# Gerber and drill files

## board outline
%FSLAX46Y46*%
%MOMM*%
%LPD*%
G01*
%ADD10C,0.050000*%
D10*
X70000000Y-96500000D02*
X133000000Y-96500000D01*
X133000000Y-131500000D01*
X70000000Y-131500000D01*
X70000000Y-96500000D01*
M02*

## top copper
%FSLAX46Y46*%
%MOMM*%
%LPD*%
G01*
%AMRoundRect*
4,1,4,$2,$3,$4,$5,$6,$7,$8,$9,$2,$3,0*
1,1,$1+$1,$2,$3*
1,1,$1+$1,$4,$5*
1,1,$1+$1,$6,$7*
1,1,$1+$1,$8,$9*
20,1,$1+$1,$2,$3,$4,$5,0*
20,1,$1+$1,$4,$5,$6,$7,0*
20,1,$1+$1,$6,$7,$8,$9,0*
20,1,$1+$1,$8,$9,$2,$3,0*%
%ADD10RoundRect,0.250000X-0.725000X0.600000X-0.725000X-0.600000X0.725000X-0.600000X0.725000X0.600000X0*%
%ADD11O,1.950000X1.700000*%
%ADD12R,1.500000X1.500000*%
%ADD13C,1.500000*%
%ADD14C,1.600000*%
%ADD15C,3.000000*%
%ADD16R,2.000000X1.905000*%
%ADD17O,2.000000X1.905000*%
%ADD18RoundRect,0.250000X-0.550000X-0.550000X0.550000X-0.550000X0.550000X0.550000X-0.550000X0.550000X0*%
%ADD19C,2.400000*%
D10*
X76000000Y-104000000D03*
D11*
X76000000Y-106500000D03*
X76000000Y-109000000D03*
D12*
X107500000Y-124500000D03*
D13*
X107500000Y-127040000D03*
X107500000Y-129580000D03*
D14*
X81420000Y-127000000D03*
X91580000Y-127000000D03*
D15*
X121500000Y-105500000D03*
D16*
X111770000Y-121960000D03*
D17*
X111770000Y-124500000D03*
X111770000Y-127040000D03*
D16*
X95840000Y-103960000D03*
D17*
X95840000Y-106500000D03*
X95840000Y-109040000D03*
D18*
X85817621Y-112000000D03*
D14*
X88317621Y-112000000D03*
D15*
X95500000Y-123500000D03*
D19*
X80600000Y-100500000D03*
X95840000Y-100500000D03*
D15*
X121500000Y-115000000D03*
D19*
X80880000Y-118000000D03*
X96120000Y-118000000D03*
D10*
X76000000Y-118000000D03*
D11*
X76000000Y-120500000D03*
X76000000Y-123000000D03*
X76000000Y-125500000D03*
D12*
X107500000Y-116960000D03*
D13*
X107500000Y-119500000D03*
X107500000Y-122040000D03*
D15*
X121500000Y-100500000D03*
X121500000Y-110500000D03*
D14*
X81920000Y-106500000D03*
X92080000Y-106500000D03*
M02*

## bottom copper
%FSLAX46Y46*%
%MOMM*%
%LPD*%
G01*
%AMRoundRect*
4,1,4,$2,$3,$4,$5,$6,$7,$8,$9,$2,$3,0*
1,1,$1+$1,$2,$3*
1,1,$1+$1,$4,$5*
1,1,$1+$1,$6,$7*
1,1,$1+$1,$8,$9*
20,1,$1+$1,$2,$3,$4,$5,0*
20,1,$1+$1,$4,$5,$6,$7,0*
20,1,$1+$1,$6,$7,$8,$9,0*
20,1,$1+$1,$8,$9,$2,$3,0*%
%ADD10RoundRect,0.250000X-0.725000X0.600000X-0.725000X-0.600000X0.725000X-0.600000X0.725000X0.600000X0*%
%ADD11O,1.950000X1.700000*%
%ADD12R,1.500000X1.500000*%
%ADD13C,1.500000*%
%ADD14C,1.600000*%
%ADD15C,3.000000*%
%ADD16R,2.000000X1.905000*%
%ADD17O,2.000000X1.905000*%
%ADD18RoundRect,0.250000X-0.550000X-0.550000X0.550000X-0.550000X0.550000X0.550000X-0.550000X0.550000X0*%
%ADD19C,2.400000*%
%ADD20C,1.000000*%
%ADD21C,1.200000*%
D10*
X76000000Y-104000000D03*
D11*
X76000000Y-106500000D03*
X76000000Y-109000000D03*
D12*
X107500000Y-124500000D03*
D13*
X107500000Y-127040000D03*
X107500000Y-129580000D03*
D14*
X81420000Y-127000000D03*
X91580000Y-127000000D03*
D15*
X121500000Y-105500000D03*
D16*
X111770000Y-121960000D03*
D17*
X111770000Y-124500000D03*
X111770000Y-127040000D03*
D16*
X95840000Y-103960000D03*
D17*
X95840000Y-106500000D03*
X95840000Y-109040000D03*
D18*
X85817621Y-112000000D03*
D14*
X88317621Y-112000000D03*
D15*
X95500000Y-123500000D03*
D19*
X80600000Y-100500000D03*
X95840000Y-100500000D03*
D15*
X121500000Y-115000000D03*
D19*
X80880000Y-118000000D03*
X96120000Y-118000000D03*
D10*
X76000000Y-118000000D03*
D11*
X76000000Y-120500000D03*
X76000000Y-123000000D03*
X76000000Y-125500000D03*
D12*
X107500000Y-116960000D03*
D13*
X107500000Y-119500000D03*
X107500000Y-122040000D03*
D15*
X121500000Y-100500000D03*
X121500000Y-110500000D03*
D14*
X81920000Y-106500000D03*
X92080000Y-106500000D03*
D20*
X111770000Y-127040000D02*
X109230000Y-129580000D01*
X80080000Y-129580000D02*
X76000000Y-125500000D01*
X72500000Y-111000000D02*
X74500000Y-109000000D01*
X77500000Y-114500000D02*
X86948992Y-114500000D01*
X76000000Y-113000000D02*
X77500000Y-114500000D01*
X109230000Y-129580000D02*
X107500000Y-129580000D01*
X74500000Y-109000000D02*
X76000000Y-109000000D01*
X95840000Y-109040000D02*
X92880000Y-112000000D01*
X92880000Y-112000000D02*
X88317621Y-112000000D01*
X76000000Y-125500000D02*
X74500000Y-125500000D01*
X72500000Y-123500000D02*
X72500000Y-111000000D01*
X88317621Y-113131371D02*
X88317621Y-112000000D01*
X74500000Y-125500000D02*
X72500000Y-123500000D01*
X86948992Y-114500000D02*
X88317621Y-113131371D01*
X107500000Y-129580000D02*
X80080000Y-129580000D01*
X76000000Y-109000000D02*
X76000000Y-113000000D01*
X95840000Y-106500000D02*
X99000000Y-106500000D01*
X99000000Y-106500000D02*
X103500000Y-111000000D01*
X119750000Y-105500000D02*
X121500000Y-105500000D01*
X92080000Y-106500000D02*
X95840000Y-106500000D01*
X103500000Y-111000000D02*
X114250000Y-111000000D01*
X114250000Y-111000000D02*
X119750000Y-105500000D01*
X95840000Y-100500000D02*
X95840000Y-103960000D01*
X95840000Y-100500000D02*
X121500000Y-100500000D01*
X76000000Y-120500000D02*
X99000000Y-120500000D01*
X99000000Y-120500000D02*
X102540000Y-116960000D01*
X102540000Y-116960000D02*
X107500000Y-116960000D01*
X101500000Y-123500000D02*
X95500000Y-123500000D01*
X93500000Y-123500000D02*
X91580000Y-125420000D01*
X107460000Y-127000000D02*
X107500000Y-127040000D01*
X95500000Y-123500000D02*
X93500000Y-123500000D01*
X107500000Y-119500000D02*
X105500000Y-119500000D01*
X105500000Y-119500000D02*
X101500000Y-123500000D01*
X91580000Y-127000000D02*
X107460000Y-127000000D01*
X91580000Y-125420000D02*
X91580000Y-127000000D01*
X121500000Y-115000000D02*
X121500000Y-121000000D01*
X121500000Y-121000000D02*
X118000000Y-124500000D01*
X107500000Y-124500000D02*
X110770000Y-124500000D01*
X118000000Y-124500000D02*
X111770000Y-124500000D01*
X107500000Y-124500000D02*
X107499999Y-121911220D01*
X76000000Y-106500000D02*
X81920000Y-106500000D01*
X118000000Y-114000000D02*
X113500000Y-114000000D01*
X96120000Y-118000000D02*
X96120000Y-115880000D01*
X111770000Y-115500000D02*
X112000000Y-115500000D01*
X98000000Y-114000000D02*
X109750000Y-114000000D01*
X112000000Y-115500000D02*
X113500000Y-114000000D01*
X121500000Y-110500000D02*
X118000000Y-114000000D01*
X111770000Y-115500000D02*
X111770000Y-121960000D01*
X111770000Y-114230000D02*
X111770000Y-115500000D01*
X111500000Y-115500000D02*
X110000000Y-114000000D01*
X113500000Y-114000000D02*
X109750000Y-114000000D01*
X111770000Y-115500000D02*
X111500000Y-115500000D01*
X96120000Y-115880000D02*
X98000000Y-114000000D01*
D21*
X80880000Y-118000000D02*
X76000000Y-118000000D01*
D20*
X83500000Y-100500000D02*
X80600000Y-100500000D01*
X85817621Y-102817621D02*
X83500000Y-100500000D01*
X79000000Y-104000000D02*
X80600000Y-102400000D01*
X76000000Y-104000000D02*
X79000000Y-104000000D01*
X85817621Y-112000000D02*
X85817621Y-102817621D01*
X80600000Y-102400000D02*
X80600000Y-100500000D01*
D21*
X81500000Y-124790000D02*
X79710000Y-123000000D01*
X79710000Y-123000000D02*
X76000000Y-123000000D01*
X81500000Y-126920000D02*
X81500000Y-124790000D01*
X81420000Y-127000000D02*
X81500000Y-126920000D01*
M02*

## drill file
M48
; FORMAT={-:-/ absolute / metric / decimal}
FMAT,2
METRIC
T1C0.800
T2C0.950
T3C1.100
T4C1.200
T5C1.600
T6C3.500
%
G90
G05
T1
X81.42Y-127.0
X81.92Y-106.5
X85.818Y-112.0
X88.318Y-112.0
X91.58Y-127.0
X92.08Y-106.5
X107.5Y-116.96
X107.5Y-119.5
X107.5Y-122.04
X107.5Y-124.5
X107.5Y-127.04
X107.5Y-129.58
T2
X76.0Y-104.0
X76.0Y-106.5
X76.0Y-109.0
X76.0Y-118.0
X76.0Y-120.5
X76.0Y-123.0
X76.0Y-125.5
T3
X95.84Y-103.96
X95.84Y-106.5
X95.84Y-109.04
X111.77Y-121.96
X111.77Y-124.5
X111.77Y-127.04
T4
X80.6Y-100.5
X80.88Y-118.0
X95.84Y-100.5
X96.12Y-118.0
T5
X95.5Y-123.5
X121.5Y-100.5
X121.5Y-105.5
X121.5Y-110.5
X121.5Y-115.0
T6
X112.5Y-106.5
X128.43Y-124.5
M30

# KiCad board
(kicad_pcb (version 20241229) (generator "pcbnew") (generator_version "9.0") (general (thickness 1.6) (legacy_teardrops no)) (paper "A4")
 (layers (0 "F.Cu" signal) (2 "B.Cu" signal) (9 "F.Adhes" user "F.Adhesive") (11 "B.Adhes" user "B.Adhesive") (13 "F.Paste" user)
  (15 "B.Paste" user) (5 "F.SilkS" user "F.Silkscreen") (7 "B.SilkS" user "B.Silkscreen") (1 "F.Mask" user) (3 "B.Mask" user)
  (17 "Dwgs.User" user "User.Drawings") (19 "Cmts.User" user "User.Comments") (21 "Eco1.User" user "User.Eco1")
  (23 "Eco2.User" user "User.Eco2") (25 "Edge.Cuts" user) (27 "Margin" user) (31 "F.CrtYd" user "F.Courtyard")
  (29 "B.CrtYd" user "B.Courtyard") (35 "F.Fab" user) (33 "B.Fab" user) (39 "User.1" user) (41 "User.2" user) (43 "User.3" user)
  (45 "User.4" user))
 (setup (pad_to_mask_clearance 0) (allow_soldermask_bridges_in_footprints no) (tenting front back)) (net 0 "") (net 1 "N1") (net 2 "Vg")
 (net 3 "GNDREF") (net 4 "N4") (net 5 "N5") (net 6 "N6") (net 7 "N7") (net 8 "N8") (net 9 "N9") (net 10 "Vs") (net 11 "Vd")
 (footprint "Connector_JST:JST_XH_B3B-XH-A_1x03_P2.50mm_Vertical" (layer "F.Cu") (at 76 104 -90)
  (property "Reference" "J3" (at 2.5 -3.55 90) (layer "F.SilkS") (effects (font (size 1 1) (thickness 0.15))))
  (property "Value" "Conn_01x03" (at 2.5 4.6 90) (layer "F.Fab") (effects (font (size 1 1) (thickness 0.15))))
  (pad "1" thru_hole roundrect (at 0 0 270) (size 1.7 1.95) (drill 0.95) (layers "*.Cu" "*.Mask") (remove_unused_layers no)
   (roundrect_rratio 0.147059) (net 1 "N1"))
  (pad "2" thru_hole oval (at 2.5 0 270) (size 1.7 1.95) (drill 0.95) (layers "*.Cu" "*.Mask") (remove_unused_layers no) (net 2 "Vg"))
  (pad "3" thru_hole oval (at 5 0 270) (size 1.7 1.95) (drill 0.95) (layers "*.Cu" "*.Mask") (remove_unused_layers no) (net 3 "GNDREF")))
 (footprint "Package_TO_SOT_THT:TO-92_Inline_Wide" (layer "F.Cu") (at 107.5 124.5 -90)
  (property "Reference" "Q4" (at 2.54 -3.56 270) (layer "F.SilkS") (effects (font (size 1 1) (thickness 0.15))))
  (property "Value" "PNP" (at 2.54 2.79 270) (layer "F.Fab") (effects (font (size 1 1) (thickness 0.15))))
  (pad "1" thru_hole rect (at 0 0 270) (size 1.5 1.5) (drill 0.8) (layers "*.Cu" "*.Mask") (remove_unused_layers no) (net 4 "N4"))
  (pad "2" thru_hole circle (at 2.54 0 270) (size 1.5 1.5) (drill 0.8) (layers "*.Cu" "*.Mask") (remove_unused_layers no) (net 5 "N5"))
  (pad "3" thru_hole circle (at 5.08 0 270) (size 1.5 1.5) (drill 0.8) (layers "*.Cu" "*.Mask") (remove_unused_layers no) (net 3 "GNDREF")))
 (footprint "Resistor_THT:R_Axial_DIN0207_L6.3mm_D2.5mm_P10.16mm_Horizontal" (layer "F.Cu") (at 81.42 127)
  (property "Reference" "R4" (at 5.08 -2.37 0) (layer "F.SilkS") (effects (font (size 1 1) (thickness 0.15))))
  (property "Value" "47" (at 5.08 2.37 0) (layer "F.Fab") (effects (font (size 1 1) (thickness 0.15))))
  (pad "1" thru_hole circle (at 0 0) (size 1.6 1.6) (drill 0.8) (layers "*.Cu" "*.Mask") (remove_unused_layers no) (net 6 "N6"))
  (pad "2" thru_hole circle (at 10.16 0) (size 1.6 1.6) (drill 0.8) (layers "*.Cu" "*.Mask") (remove_unused_layers no) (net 5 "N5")))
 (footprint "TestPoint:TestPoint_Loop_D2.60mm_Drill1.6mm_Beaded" (layer "F.Cu") (at 121.5 105.5)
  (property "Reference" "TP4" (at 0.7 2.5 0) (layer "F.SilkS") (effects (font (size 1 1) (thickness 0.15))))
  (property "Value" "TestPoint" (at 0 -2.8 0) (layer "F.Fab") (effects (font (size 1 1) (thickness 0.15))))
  (pad "1" thru_hole circle (at 0 0) (size 3 3) (drill 1.6) (layers "*.Cu" "*.Mask") (remove_unused_layers no) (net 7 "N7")))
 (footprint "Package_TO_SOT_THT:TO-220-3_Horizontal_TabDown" (layer "F.Cu") (at 111.77 121.96 -90)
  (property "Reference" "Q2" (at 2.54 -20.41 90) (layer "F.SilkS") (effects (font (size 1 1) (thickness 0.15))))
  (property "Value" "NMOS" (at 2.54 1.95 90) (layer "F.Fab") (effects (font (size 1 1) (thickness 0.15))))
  (pad "" np_thru_hole circle (at 2.54 -16.66 270) (size 3.5 3.5) (drill 3.5) (layers "*.Cu" "*.Mask"))
  (pad "1" thru_hole rect (at 0 0 270) (size 1.905 2) (drill 1.1) (layers "*.Cu" "*.Mask") (remove_unused_layers no) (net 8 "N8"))
  (pad "2" thru_hole oval (at 2.54 0 270) (size 1.905 2) (drill 1.1) (layers "*.Cu" "*.Mask") (remove_unused_layers no) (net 4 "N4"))
  (pad "3" thru_hole oval (at 5.08 0 270) (size 1.905 2) (drill 1.1) (layers "*.Cu" "*.Mask") (remove_unused_layers no) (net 3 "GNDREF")))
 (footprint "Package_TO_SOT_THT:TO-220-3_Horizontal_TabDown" (layer "F.Cu") (at 95.84 103.96 -90)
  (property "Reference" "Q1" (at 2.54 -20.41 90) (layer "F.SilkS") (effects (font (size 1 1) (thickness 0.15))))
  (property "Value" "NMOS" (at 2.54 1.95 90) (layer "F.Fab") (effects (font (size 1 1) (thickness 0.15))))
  (pad "" np_thru_hole circle (at 2.54 -16.66 270) (size 3.5 3.5) (drill 3.5) (layers "*.Cu" "*.Mask"))
  (pad "1" thru_hole rect (at 0 0 270) (size 1.905 2) (drill 1.1) (layers "*.Cu" "*.Mask") (remove_unused_layers no) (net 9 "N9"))
  (pad "2" thru_hole oval (at 2.54 0 270) (size 1.905 2) (drill 1.1) (layers "*.Cu" "*.Mask") (remove_unused_layers no) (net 7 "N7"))
  (pad "3" thru_hole oval (at 5.08 0 270) (size 1.905 2) (drill 1.1) (layers "*.Cu" "*.Mask") (remove_unused_layers no) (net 3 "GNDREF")))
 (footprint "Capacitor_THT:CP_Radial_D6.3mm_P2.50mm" (layer "F.Cu") (at 85.817621 112)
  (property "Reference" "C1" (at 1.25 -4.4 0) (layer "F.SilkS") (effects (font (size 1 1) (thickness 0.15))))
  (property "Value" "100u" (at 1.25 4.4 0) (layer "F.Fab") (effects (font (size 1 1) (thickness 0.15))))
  (pad "1" thru_hole roundrect (at 0 0) (size 1.6 1.6) (drill 0.8) (layers "*.Cu" "*.Mask") (remove_unused_layers no)
   (roundrect_rratio 0.15625) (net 1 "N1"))
  (pad "2" thru_hole circle (at 2.5 0) (size 1.6 1.6) (drill 0.8) (layers "*.Cu" "*.Mask") (remove_unused_layers no) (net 3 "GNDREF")))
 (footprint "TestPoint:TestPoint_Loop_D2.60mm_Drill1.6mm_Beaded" (layer "F.Cu") (at 95.5 123.5)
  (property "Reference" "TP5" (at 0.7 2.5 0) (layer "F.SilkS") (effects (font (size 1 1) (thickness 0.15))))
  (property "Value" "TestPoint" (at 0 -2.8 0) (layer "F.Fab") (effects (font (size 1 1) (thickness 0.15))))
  (pad "1" thru_hole circle (at 0 0) (size 3 3) (drill 1.6) (layers "*.Cu" "*.Mask") (remove_unused_layers no) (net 5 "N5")))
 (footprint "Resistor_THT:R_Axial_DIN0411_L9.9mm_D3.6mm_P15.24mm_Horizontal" (layer "F.Cu") (at 80.6 100.5)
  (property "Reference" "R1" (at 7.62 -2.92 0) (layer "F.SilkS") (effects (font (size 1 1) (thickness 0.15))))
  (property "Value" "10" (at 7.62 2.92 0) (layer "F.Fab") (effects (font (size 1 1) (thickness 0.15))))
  (pad "1" thru_hole circle (at 0 0) (size 2.4 2.4) (drill 1.2) (layers "*.Cu" "*.Mask") (remove_unused_layers no) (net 1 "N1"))
  (pad "2" thru_hole circle (at 15.24 0) (size 2.4 2.4) (drill 1.2) (layers "*.Cu" "*.Mask") (remove_unused_layers no) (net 9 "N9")))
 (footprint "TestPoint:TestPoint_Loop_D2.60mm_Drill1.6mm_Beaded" (layer "F.Cu") (at 121.5 115)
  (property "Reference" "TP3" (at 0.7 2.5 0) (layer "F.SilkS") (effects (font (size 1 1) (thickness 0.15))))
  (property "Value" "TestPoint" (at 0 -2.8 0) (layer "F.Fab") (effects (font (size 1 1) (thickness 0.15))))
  (pad "1" thru_hole circle (at 0 0) (size 3 3) (drill 1.6) (layers "*.Cu" "*.Mask") (remove_unused_layers no) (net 4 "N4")))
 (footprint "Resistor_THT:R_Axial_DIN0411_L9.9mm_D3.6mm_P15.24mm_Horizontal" (layer "F.Cu") (at 80.88 118)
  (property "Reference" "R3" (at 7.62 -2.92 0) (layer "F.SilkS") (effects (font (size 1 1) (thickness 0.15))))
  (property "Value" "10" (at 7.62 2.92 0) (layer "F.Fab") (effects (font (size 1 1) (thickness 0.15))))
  (pad "1" thru_hole circle (at 0 0) (size 2.4 2.4) (drill 1.2) (layers "*.Cu" "*.Mask") (remove_unused_layers no) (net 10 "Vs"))
  (pad "2" thru_hole circle (at 15.24 0) (size 2.4 2.4) (drill 1.2) (layers "*.Cu" "*.Mask") (remove_unused_layers no) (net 8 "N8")))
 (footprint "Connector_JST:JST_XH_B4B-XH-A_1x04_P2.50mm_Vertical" (layer "F.Cu") (at 76 118 -90)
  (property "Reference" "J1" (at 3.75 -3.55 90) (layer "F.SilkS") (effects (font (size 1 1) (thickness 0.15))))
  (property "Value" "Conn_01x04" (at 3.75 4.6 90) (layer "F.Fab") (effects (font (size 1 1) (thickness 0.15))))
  (pad "1" thru_hole roundrect (at 0 0 270) (size 1.7 1.95) (drill 0.95) (layers "*.Cu" "*.Mask") (remove_unused_layers no)
   (roundrect_rratio 0.147059) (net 10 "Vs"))
  (pad "2" thru_hole oval (at 2.5 0 270) (size 1.7 1.95) (drill 0.95) (layers "*.Cu" "*.Mask") (remove_unused_layers no) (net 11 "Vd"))
  (pad "3" thru_hole oval (at 5 0 270) (size 1.7 1.95) (drill 0.95) (layers "*.Cu" "*.Mask") (remove_unused_layers no) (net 6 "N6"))
  (pad "4" thru_hole oval (at 7.5 0 270) (size 1.7 1.95) (drill 0.95) (layers "*.Cu" "*.Mask") (remove_unused_layers no) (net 3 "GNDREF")))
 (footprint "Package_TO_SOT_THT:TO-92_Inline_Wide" (layer "F.Cu") (at 107.5 116.96 -90)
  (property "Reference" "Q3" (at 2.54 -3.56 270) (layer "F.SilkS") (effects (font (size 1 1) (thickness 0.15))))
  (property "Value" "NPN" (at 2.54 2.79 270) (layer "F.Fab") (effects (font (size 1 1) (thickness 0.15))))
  (pad "1" thru_hole rect (at 0 0 270) (size 1.5 1.5) (drill 0.8) (layers "*.Cu" "*.Mask") (remove_unused_layers no) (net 11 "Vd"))
  (pad "2" thru_hole circle (at 2.54 0 270) (size 1.5 1.5) (drill 0.8) (layers "*.Cu" "*.Mask") (remove_unused_layers no) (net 5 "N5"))
  (pad "3" thru_hole circle (at 5.08 0 270) (size 1.5 1.5) (drill 0.8) (layers "*.Cu" "*.Mask") (remove_unused_layers no) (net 4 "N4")))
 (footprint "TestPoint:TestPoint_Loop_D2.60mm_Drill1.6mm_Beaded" (layer "F.Cu") (at 121.5 100.5)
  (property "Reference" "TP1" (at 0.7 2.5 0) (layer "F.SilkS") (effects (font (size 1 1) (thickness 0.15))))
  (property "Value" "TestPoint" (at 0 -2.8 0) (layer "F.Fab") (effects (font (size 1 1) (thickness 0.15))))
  (pad "1" thru_hole circle (at 0 0) (size 3 3) (drill 1.6) (layers "*.Cu" "*.Mask") (remove_unused_layers no) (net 9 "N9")))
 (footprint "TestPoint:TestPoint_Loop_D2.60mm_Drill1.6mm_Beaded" (layer "F.Cu") (at 121.5 110.5)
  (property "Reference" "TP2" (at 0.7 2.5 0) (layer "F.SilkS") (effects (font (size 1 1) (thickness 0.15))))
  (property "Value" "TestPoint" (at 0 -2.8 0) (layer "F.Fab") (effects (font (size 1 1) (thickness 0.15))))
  (pad "1" thru_hole circle (at 0 0) (size 3 3) (drill 1.6) (layers "*.Cu" "*.Mask") (remove_unused_layers no) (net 8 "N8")))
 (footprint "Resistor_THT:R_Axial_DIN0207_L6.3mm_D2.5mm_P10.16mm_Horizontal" (layer "F.Cu") (at 81.92 106.5)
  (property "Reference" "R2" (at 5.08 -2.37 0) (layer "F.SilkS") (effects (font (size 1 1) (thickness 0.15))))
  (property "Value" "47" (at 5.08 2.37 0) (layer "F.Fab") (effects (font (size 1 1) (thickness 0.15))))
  (pad "1" thru_hole circle (at 0 0) (size 1.6 1.6) (drill 0.8) (layers "*.Cu" "*.Mask") (remove_unused_layers no) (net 2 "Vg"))
  (pad "2" thru_hole circle (at 10.16 0) (size 1.6 1.6) (drill 0.8) (layers "*.Cu" "*.Mask") (remove_unused_layers no) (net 7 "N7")))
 (gr_rect (start 70 96.5) (end 133 131.5) (stroke (width 0.05) (type default)) (fill no) (layer "Edge.Cuts"))
 (segment (start 111.77 127.04) (end 109.23 129.58) (width 1) (layer "B.Cu") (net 3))
 (segment (start 80.08 129.58) (end 76 125.5) (width 1) (layer "B.Cu") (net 3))
 (segment (start 72.5 111) (end 74.5 109) (width 1) (layer "B.Cu") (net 3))
 (segment (start 77.5 114.5) (end 86.948992 114.5) (width 1) (layer "B.Cu") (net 3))
 (segment (start 76 113) (end 77.5 114.5) (width 1) (layer "B.Cu") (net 3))
 (segment (start 109.23 129.58) (end 107.5 129.58) (width 1) (layer "B.Cu") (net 3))
 (segment (start 74.5 109) (end 76 109) (width 1) (layer "B.Cu") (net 3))
 (segment (start 95.84 109.04) (end 92.88 112) (width 1) (layer "B.Cu") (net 3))
 (segment (start 92.88 112) (end 88.317621 112) (width 1) (layer "B.Cu") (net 3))
 (segment (start 76 125.5) (end 74.5 125.5) (width 1) (layer "B.Cu") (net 3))
 (segment (start 72.5 123.5) (end 72.5 111) (width 1) (layer "B.Cu") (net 3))
 (segment (start 88.317621 113.131371) (end 88.317621 112) (width 1) (layer "B.Cu") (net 3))
 (segment (start 74.5 125.5) (end 72.5 123.5) (width 1) (layer "B.Cu") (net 3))
 (segment (start 86.948992 114.5) (end 88.317621 113.131371) (width 1) (layer "B.Cu") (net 3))
 (segment (start 107.5 129.58) (end 80.08 129.58) (width 1) (layer "B.Cu") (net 3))
 (segment (start 76 109) (end 76 113) (width 1) (layer "B.Cu") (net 3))
 (segment (start 95.84 106.5) (end 99 106.5) (width 1) (layer "B.Cu") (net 7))
 (segment (start 99 106.5) (end 103.5 111) (width 1) (layer "B.Cu") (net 7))
 (segment (start 119.75 105.5) (end 121.5 105.5) (width 1) (layer "B.Cu") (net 7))
 (segment (start 92.08 106.5) (end 95.84 106.5) (width 1) (layer "B.Cu") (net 7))
 (segment (start 103.5 111) (end 114.25 111) (width 1) (layer "B.Cu") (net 7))
 (segment (start 114.25 111) (end 119.75 105.5) (width 1) (layer "B.Cu") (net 7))
 (segment (start 95.84 100.5) (end 95.84 103.96) (width 1) (layer "B.Cu") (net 9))
 (segment (start 95.84 100.5) (end 121.5 100.5) (width 1) (layer "B.Cu") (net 9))
 (segment (start 76 120.5) (end 99 120.5) (width 1) (layer "B.Cu") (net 11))
 (segment (start 99 120.5) (end 102.54 116.96) (width 1) (layer "B.Cu") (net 11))
 (segment (start 102.54 116.96) (end 107.5 116.96) (width 1) (layer "B.Cu") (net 11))
 (segment (start 101.5 123.5) (end 95.5 123.5) (width 1) (layer "B.Cu") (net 5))
 (segment (start 93.5 123.5) (end 91.58 125.42) (width 1) (layer "B.Cu") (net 5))
 (segment (start 107.46 127) (end 107.5 127.04) (width 1) (layer "B.Cu") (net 5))
 (segment (start 95.5 123.5) (end 93.5 123.5) (width 1) (layer "B.Cu") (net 5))
 (segment (start 107.5 119.5) (end 105.5 119.5) (width 1) (layer "B.Cu") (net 5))
 (segment (start 105.5 119.5) (end 101.5 123.5) (width 1) (layer "B.Cu") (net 5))
 (segment (start 91.58 127) (end 107.46 127) (width 1) (layer "B.Cu") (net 5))
 (segment (start 91.58 125.42) (end 91.58 127) (width 1) (layer "B.Cu") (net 5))
 (segment (start 121.5 115) (end 121.5 121) (width 1) (layer "B.Cu") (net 4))
 (segment (start 121.5 121) (end 118 124.5) (width 1) (layer "B.Cu") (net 4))
 (segment (start 107.5 124.5) (end 110.77 124.5) (width 1) (layer "B.Cu") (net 4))
 (segment (start 118 124.5) (end 111.77 124.5) (width 1) (layer "B.Cu") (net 4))
 (segment (start 107.5 124.5) (end 107.499999 121.91122) (width 1) (layer "B.Cu") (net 4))
 (segment (start 76 106.5) (end 81.92 106.5) (width 1) (layer "B.Cu") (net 2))
 (segment (start 118 114) (end 113.5 114) (width 1) (layer "B.Cu") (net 8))
 (segment (start 96.12 118) (end 96.12 115.88) (width 1) (layer "B.Cu") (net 8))
 (segment (start 111.77 115.5) (end 112 115.5) (width 1) (layer "B.Cu") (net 8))
 (segment (start 98 114) (end 109.75 114) (width 1) (layer "B.Cu") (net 8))
 (segment (start 112 115.5) (end 113.5 114) (width 1) (layer "B.Cu") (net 8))
 (segment (start 121.5 110.5) (end 118 114) (width 1) (layer "B.Cu") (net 8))
 (segment (start 111.77 115.5) (end 111.77 121.96) (width 1) (layer "B.Cu") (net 8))
 (segment (start 111.77 114.23) (end 111.77 115.5) (width 1) (layer "B.Cu") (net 8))
 (segment (start 111.5 115.5) (end 110 114) (width 1) (layer "B.Cu") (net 8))
 (segment (start 113.5 114) (end 109.75 114) (width 1) (layer "B.Cu") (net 8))
 (segment (start 111.77 115.5) (end 111.5 115.5) (width 1) (layer "B.Cu") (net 8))
 (segment (start 96.12 115.88) (end 98 114) (width 1) (layer "B.Cu") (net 8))
 (segment (start 80.88 118) (end 76 118) (width 1.2) (layer "B.Cu") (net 10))
 (segment (start 83.5 100.5) (end 80.6 100.5) (width 1) (layer "B.Cu") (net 1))
 (segment (start 85.817621 102.817621) (end 83.5 100.5) (width 1) (layer "B.Cu") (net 1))
 (segment (start 79 104) (end 80.6 102.4) (width 1) (layer "B.Cu") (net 1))
 (segment (start 76 104) (end 79 104) (width 1) (layer "B.Cu") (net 1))
 (segment (start 85.817621 112) (end 85.817621 102.817621) (width 1) (layer "B.Cu") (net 1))
 (segment (start 80.6 102.4) (end 80.6 100.5) (width 1) (layer "B.Cu") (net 1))
 (segment (start 81.5 124.79) (end 79.71 123) (width 1.2) (layer "B.Cu") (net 6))
 (segment (start 79.71 123) (end 76 123) (width 1.2) (layer "B.Cu") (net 6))
 (segment (start 81.5 126.92) (end 81.5 124.79) (width 1.2) (layer "B.Cu") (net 6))
 (segment (start 81.42 127) (end 81.5 126.92) (width 1.2) (layer "B.Cu") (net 6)))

